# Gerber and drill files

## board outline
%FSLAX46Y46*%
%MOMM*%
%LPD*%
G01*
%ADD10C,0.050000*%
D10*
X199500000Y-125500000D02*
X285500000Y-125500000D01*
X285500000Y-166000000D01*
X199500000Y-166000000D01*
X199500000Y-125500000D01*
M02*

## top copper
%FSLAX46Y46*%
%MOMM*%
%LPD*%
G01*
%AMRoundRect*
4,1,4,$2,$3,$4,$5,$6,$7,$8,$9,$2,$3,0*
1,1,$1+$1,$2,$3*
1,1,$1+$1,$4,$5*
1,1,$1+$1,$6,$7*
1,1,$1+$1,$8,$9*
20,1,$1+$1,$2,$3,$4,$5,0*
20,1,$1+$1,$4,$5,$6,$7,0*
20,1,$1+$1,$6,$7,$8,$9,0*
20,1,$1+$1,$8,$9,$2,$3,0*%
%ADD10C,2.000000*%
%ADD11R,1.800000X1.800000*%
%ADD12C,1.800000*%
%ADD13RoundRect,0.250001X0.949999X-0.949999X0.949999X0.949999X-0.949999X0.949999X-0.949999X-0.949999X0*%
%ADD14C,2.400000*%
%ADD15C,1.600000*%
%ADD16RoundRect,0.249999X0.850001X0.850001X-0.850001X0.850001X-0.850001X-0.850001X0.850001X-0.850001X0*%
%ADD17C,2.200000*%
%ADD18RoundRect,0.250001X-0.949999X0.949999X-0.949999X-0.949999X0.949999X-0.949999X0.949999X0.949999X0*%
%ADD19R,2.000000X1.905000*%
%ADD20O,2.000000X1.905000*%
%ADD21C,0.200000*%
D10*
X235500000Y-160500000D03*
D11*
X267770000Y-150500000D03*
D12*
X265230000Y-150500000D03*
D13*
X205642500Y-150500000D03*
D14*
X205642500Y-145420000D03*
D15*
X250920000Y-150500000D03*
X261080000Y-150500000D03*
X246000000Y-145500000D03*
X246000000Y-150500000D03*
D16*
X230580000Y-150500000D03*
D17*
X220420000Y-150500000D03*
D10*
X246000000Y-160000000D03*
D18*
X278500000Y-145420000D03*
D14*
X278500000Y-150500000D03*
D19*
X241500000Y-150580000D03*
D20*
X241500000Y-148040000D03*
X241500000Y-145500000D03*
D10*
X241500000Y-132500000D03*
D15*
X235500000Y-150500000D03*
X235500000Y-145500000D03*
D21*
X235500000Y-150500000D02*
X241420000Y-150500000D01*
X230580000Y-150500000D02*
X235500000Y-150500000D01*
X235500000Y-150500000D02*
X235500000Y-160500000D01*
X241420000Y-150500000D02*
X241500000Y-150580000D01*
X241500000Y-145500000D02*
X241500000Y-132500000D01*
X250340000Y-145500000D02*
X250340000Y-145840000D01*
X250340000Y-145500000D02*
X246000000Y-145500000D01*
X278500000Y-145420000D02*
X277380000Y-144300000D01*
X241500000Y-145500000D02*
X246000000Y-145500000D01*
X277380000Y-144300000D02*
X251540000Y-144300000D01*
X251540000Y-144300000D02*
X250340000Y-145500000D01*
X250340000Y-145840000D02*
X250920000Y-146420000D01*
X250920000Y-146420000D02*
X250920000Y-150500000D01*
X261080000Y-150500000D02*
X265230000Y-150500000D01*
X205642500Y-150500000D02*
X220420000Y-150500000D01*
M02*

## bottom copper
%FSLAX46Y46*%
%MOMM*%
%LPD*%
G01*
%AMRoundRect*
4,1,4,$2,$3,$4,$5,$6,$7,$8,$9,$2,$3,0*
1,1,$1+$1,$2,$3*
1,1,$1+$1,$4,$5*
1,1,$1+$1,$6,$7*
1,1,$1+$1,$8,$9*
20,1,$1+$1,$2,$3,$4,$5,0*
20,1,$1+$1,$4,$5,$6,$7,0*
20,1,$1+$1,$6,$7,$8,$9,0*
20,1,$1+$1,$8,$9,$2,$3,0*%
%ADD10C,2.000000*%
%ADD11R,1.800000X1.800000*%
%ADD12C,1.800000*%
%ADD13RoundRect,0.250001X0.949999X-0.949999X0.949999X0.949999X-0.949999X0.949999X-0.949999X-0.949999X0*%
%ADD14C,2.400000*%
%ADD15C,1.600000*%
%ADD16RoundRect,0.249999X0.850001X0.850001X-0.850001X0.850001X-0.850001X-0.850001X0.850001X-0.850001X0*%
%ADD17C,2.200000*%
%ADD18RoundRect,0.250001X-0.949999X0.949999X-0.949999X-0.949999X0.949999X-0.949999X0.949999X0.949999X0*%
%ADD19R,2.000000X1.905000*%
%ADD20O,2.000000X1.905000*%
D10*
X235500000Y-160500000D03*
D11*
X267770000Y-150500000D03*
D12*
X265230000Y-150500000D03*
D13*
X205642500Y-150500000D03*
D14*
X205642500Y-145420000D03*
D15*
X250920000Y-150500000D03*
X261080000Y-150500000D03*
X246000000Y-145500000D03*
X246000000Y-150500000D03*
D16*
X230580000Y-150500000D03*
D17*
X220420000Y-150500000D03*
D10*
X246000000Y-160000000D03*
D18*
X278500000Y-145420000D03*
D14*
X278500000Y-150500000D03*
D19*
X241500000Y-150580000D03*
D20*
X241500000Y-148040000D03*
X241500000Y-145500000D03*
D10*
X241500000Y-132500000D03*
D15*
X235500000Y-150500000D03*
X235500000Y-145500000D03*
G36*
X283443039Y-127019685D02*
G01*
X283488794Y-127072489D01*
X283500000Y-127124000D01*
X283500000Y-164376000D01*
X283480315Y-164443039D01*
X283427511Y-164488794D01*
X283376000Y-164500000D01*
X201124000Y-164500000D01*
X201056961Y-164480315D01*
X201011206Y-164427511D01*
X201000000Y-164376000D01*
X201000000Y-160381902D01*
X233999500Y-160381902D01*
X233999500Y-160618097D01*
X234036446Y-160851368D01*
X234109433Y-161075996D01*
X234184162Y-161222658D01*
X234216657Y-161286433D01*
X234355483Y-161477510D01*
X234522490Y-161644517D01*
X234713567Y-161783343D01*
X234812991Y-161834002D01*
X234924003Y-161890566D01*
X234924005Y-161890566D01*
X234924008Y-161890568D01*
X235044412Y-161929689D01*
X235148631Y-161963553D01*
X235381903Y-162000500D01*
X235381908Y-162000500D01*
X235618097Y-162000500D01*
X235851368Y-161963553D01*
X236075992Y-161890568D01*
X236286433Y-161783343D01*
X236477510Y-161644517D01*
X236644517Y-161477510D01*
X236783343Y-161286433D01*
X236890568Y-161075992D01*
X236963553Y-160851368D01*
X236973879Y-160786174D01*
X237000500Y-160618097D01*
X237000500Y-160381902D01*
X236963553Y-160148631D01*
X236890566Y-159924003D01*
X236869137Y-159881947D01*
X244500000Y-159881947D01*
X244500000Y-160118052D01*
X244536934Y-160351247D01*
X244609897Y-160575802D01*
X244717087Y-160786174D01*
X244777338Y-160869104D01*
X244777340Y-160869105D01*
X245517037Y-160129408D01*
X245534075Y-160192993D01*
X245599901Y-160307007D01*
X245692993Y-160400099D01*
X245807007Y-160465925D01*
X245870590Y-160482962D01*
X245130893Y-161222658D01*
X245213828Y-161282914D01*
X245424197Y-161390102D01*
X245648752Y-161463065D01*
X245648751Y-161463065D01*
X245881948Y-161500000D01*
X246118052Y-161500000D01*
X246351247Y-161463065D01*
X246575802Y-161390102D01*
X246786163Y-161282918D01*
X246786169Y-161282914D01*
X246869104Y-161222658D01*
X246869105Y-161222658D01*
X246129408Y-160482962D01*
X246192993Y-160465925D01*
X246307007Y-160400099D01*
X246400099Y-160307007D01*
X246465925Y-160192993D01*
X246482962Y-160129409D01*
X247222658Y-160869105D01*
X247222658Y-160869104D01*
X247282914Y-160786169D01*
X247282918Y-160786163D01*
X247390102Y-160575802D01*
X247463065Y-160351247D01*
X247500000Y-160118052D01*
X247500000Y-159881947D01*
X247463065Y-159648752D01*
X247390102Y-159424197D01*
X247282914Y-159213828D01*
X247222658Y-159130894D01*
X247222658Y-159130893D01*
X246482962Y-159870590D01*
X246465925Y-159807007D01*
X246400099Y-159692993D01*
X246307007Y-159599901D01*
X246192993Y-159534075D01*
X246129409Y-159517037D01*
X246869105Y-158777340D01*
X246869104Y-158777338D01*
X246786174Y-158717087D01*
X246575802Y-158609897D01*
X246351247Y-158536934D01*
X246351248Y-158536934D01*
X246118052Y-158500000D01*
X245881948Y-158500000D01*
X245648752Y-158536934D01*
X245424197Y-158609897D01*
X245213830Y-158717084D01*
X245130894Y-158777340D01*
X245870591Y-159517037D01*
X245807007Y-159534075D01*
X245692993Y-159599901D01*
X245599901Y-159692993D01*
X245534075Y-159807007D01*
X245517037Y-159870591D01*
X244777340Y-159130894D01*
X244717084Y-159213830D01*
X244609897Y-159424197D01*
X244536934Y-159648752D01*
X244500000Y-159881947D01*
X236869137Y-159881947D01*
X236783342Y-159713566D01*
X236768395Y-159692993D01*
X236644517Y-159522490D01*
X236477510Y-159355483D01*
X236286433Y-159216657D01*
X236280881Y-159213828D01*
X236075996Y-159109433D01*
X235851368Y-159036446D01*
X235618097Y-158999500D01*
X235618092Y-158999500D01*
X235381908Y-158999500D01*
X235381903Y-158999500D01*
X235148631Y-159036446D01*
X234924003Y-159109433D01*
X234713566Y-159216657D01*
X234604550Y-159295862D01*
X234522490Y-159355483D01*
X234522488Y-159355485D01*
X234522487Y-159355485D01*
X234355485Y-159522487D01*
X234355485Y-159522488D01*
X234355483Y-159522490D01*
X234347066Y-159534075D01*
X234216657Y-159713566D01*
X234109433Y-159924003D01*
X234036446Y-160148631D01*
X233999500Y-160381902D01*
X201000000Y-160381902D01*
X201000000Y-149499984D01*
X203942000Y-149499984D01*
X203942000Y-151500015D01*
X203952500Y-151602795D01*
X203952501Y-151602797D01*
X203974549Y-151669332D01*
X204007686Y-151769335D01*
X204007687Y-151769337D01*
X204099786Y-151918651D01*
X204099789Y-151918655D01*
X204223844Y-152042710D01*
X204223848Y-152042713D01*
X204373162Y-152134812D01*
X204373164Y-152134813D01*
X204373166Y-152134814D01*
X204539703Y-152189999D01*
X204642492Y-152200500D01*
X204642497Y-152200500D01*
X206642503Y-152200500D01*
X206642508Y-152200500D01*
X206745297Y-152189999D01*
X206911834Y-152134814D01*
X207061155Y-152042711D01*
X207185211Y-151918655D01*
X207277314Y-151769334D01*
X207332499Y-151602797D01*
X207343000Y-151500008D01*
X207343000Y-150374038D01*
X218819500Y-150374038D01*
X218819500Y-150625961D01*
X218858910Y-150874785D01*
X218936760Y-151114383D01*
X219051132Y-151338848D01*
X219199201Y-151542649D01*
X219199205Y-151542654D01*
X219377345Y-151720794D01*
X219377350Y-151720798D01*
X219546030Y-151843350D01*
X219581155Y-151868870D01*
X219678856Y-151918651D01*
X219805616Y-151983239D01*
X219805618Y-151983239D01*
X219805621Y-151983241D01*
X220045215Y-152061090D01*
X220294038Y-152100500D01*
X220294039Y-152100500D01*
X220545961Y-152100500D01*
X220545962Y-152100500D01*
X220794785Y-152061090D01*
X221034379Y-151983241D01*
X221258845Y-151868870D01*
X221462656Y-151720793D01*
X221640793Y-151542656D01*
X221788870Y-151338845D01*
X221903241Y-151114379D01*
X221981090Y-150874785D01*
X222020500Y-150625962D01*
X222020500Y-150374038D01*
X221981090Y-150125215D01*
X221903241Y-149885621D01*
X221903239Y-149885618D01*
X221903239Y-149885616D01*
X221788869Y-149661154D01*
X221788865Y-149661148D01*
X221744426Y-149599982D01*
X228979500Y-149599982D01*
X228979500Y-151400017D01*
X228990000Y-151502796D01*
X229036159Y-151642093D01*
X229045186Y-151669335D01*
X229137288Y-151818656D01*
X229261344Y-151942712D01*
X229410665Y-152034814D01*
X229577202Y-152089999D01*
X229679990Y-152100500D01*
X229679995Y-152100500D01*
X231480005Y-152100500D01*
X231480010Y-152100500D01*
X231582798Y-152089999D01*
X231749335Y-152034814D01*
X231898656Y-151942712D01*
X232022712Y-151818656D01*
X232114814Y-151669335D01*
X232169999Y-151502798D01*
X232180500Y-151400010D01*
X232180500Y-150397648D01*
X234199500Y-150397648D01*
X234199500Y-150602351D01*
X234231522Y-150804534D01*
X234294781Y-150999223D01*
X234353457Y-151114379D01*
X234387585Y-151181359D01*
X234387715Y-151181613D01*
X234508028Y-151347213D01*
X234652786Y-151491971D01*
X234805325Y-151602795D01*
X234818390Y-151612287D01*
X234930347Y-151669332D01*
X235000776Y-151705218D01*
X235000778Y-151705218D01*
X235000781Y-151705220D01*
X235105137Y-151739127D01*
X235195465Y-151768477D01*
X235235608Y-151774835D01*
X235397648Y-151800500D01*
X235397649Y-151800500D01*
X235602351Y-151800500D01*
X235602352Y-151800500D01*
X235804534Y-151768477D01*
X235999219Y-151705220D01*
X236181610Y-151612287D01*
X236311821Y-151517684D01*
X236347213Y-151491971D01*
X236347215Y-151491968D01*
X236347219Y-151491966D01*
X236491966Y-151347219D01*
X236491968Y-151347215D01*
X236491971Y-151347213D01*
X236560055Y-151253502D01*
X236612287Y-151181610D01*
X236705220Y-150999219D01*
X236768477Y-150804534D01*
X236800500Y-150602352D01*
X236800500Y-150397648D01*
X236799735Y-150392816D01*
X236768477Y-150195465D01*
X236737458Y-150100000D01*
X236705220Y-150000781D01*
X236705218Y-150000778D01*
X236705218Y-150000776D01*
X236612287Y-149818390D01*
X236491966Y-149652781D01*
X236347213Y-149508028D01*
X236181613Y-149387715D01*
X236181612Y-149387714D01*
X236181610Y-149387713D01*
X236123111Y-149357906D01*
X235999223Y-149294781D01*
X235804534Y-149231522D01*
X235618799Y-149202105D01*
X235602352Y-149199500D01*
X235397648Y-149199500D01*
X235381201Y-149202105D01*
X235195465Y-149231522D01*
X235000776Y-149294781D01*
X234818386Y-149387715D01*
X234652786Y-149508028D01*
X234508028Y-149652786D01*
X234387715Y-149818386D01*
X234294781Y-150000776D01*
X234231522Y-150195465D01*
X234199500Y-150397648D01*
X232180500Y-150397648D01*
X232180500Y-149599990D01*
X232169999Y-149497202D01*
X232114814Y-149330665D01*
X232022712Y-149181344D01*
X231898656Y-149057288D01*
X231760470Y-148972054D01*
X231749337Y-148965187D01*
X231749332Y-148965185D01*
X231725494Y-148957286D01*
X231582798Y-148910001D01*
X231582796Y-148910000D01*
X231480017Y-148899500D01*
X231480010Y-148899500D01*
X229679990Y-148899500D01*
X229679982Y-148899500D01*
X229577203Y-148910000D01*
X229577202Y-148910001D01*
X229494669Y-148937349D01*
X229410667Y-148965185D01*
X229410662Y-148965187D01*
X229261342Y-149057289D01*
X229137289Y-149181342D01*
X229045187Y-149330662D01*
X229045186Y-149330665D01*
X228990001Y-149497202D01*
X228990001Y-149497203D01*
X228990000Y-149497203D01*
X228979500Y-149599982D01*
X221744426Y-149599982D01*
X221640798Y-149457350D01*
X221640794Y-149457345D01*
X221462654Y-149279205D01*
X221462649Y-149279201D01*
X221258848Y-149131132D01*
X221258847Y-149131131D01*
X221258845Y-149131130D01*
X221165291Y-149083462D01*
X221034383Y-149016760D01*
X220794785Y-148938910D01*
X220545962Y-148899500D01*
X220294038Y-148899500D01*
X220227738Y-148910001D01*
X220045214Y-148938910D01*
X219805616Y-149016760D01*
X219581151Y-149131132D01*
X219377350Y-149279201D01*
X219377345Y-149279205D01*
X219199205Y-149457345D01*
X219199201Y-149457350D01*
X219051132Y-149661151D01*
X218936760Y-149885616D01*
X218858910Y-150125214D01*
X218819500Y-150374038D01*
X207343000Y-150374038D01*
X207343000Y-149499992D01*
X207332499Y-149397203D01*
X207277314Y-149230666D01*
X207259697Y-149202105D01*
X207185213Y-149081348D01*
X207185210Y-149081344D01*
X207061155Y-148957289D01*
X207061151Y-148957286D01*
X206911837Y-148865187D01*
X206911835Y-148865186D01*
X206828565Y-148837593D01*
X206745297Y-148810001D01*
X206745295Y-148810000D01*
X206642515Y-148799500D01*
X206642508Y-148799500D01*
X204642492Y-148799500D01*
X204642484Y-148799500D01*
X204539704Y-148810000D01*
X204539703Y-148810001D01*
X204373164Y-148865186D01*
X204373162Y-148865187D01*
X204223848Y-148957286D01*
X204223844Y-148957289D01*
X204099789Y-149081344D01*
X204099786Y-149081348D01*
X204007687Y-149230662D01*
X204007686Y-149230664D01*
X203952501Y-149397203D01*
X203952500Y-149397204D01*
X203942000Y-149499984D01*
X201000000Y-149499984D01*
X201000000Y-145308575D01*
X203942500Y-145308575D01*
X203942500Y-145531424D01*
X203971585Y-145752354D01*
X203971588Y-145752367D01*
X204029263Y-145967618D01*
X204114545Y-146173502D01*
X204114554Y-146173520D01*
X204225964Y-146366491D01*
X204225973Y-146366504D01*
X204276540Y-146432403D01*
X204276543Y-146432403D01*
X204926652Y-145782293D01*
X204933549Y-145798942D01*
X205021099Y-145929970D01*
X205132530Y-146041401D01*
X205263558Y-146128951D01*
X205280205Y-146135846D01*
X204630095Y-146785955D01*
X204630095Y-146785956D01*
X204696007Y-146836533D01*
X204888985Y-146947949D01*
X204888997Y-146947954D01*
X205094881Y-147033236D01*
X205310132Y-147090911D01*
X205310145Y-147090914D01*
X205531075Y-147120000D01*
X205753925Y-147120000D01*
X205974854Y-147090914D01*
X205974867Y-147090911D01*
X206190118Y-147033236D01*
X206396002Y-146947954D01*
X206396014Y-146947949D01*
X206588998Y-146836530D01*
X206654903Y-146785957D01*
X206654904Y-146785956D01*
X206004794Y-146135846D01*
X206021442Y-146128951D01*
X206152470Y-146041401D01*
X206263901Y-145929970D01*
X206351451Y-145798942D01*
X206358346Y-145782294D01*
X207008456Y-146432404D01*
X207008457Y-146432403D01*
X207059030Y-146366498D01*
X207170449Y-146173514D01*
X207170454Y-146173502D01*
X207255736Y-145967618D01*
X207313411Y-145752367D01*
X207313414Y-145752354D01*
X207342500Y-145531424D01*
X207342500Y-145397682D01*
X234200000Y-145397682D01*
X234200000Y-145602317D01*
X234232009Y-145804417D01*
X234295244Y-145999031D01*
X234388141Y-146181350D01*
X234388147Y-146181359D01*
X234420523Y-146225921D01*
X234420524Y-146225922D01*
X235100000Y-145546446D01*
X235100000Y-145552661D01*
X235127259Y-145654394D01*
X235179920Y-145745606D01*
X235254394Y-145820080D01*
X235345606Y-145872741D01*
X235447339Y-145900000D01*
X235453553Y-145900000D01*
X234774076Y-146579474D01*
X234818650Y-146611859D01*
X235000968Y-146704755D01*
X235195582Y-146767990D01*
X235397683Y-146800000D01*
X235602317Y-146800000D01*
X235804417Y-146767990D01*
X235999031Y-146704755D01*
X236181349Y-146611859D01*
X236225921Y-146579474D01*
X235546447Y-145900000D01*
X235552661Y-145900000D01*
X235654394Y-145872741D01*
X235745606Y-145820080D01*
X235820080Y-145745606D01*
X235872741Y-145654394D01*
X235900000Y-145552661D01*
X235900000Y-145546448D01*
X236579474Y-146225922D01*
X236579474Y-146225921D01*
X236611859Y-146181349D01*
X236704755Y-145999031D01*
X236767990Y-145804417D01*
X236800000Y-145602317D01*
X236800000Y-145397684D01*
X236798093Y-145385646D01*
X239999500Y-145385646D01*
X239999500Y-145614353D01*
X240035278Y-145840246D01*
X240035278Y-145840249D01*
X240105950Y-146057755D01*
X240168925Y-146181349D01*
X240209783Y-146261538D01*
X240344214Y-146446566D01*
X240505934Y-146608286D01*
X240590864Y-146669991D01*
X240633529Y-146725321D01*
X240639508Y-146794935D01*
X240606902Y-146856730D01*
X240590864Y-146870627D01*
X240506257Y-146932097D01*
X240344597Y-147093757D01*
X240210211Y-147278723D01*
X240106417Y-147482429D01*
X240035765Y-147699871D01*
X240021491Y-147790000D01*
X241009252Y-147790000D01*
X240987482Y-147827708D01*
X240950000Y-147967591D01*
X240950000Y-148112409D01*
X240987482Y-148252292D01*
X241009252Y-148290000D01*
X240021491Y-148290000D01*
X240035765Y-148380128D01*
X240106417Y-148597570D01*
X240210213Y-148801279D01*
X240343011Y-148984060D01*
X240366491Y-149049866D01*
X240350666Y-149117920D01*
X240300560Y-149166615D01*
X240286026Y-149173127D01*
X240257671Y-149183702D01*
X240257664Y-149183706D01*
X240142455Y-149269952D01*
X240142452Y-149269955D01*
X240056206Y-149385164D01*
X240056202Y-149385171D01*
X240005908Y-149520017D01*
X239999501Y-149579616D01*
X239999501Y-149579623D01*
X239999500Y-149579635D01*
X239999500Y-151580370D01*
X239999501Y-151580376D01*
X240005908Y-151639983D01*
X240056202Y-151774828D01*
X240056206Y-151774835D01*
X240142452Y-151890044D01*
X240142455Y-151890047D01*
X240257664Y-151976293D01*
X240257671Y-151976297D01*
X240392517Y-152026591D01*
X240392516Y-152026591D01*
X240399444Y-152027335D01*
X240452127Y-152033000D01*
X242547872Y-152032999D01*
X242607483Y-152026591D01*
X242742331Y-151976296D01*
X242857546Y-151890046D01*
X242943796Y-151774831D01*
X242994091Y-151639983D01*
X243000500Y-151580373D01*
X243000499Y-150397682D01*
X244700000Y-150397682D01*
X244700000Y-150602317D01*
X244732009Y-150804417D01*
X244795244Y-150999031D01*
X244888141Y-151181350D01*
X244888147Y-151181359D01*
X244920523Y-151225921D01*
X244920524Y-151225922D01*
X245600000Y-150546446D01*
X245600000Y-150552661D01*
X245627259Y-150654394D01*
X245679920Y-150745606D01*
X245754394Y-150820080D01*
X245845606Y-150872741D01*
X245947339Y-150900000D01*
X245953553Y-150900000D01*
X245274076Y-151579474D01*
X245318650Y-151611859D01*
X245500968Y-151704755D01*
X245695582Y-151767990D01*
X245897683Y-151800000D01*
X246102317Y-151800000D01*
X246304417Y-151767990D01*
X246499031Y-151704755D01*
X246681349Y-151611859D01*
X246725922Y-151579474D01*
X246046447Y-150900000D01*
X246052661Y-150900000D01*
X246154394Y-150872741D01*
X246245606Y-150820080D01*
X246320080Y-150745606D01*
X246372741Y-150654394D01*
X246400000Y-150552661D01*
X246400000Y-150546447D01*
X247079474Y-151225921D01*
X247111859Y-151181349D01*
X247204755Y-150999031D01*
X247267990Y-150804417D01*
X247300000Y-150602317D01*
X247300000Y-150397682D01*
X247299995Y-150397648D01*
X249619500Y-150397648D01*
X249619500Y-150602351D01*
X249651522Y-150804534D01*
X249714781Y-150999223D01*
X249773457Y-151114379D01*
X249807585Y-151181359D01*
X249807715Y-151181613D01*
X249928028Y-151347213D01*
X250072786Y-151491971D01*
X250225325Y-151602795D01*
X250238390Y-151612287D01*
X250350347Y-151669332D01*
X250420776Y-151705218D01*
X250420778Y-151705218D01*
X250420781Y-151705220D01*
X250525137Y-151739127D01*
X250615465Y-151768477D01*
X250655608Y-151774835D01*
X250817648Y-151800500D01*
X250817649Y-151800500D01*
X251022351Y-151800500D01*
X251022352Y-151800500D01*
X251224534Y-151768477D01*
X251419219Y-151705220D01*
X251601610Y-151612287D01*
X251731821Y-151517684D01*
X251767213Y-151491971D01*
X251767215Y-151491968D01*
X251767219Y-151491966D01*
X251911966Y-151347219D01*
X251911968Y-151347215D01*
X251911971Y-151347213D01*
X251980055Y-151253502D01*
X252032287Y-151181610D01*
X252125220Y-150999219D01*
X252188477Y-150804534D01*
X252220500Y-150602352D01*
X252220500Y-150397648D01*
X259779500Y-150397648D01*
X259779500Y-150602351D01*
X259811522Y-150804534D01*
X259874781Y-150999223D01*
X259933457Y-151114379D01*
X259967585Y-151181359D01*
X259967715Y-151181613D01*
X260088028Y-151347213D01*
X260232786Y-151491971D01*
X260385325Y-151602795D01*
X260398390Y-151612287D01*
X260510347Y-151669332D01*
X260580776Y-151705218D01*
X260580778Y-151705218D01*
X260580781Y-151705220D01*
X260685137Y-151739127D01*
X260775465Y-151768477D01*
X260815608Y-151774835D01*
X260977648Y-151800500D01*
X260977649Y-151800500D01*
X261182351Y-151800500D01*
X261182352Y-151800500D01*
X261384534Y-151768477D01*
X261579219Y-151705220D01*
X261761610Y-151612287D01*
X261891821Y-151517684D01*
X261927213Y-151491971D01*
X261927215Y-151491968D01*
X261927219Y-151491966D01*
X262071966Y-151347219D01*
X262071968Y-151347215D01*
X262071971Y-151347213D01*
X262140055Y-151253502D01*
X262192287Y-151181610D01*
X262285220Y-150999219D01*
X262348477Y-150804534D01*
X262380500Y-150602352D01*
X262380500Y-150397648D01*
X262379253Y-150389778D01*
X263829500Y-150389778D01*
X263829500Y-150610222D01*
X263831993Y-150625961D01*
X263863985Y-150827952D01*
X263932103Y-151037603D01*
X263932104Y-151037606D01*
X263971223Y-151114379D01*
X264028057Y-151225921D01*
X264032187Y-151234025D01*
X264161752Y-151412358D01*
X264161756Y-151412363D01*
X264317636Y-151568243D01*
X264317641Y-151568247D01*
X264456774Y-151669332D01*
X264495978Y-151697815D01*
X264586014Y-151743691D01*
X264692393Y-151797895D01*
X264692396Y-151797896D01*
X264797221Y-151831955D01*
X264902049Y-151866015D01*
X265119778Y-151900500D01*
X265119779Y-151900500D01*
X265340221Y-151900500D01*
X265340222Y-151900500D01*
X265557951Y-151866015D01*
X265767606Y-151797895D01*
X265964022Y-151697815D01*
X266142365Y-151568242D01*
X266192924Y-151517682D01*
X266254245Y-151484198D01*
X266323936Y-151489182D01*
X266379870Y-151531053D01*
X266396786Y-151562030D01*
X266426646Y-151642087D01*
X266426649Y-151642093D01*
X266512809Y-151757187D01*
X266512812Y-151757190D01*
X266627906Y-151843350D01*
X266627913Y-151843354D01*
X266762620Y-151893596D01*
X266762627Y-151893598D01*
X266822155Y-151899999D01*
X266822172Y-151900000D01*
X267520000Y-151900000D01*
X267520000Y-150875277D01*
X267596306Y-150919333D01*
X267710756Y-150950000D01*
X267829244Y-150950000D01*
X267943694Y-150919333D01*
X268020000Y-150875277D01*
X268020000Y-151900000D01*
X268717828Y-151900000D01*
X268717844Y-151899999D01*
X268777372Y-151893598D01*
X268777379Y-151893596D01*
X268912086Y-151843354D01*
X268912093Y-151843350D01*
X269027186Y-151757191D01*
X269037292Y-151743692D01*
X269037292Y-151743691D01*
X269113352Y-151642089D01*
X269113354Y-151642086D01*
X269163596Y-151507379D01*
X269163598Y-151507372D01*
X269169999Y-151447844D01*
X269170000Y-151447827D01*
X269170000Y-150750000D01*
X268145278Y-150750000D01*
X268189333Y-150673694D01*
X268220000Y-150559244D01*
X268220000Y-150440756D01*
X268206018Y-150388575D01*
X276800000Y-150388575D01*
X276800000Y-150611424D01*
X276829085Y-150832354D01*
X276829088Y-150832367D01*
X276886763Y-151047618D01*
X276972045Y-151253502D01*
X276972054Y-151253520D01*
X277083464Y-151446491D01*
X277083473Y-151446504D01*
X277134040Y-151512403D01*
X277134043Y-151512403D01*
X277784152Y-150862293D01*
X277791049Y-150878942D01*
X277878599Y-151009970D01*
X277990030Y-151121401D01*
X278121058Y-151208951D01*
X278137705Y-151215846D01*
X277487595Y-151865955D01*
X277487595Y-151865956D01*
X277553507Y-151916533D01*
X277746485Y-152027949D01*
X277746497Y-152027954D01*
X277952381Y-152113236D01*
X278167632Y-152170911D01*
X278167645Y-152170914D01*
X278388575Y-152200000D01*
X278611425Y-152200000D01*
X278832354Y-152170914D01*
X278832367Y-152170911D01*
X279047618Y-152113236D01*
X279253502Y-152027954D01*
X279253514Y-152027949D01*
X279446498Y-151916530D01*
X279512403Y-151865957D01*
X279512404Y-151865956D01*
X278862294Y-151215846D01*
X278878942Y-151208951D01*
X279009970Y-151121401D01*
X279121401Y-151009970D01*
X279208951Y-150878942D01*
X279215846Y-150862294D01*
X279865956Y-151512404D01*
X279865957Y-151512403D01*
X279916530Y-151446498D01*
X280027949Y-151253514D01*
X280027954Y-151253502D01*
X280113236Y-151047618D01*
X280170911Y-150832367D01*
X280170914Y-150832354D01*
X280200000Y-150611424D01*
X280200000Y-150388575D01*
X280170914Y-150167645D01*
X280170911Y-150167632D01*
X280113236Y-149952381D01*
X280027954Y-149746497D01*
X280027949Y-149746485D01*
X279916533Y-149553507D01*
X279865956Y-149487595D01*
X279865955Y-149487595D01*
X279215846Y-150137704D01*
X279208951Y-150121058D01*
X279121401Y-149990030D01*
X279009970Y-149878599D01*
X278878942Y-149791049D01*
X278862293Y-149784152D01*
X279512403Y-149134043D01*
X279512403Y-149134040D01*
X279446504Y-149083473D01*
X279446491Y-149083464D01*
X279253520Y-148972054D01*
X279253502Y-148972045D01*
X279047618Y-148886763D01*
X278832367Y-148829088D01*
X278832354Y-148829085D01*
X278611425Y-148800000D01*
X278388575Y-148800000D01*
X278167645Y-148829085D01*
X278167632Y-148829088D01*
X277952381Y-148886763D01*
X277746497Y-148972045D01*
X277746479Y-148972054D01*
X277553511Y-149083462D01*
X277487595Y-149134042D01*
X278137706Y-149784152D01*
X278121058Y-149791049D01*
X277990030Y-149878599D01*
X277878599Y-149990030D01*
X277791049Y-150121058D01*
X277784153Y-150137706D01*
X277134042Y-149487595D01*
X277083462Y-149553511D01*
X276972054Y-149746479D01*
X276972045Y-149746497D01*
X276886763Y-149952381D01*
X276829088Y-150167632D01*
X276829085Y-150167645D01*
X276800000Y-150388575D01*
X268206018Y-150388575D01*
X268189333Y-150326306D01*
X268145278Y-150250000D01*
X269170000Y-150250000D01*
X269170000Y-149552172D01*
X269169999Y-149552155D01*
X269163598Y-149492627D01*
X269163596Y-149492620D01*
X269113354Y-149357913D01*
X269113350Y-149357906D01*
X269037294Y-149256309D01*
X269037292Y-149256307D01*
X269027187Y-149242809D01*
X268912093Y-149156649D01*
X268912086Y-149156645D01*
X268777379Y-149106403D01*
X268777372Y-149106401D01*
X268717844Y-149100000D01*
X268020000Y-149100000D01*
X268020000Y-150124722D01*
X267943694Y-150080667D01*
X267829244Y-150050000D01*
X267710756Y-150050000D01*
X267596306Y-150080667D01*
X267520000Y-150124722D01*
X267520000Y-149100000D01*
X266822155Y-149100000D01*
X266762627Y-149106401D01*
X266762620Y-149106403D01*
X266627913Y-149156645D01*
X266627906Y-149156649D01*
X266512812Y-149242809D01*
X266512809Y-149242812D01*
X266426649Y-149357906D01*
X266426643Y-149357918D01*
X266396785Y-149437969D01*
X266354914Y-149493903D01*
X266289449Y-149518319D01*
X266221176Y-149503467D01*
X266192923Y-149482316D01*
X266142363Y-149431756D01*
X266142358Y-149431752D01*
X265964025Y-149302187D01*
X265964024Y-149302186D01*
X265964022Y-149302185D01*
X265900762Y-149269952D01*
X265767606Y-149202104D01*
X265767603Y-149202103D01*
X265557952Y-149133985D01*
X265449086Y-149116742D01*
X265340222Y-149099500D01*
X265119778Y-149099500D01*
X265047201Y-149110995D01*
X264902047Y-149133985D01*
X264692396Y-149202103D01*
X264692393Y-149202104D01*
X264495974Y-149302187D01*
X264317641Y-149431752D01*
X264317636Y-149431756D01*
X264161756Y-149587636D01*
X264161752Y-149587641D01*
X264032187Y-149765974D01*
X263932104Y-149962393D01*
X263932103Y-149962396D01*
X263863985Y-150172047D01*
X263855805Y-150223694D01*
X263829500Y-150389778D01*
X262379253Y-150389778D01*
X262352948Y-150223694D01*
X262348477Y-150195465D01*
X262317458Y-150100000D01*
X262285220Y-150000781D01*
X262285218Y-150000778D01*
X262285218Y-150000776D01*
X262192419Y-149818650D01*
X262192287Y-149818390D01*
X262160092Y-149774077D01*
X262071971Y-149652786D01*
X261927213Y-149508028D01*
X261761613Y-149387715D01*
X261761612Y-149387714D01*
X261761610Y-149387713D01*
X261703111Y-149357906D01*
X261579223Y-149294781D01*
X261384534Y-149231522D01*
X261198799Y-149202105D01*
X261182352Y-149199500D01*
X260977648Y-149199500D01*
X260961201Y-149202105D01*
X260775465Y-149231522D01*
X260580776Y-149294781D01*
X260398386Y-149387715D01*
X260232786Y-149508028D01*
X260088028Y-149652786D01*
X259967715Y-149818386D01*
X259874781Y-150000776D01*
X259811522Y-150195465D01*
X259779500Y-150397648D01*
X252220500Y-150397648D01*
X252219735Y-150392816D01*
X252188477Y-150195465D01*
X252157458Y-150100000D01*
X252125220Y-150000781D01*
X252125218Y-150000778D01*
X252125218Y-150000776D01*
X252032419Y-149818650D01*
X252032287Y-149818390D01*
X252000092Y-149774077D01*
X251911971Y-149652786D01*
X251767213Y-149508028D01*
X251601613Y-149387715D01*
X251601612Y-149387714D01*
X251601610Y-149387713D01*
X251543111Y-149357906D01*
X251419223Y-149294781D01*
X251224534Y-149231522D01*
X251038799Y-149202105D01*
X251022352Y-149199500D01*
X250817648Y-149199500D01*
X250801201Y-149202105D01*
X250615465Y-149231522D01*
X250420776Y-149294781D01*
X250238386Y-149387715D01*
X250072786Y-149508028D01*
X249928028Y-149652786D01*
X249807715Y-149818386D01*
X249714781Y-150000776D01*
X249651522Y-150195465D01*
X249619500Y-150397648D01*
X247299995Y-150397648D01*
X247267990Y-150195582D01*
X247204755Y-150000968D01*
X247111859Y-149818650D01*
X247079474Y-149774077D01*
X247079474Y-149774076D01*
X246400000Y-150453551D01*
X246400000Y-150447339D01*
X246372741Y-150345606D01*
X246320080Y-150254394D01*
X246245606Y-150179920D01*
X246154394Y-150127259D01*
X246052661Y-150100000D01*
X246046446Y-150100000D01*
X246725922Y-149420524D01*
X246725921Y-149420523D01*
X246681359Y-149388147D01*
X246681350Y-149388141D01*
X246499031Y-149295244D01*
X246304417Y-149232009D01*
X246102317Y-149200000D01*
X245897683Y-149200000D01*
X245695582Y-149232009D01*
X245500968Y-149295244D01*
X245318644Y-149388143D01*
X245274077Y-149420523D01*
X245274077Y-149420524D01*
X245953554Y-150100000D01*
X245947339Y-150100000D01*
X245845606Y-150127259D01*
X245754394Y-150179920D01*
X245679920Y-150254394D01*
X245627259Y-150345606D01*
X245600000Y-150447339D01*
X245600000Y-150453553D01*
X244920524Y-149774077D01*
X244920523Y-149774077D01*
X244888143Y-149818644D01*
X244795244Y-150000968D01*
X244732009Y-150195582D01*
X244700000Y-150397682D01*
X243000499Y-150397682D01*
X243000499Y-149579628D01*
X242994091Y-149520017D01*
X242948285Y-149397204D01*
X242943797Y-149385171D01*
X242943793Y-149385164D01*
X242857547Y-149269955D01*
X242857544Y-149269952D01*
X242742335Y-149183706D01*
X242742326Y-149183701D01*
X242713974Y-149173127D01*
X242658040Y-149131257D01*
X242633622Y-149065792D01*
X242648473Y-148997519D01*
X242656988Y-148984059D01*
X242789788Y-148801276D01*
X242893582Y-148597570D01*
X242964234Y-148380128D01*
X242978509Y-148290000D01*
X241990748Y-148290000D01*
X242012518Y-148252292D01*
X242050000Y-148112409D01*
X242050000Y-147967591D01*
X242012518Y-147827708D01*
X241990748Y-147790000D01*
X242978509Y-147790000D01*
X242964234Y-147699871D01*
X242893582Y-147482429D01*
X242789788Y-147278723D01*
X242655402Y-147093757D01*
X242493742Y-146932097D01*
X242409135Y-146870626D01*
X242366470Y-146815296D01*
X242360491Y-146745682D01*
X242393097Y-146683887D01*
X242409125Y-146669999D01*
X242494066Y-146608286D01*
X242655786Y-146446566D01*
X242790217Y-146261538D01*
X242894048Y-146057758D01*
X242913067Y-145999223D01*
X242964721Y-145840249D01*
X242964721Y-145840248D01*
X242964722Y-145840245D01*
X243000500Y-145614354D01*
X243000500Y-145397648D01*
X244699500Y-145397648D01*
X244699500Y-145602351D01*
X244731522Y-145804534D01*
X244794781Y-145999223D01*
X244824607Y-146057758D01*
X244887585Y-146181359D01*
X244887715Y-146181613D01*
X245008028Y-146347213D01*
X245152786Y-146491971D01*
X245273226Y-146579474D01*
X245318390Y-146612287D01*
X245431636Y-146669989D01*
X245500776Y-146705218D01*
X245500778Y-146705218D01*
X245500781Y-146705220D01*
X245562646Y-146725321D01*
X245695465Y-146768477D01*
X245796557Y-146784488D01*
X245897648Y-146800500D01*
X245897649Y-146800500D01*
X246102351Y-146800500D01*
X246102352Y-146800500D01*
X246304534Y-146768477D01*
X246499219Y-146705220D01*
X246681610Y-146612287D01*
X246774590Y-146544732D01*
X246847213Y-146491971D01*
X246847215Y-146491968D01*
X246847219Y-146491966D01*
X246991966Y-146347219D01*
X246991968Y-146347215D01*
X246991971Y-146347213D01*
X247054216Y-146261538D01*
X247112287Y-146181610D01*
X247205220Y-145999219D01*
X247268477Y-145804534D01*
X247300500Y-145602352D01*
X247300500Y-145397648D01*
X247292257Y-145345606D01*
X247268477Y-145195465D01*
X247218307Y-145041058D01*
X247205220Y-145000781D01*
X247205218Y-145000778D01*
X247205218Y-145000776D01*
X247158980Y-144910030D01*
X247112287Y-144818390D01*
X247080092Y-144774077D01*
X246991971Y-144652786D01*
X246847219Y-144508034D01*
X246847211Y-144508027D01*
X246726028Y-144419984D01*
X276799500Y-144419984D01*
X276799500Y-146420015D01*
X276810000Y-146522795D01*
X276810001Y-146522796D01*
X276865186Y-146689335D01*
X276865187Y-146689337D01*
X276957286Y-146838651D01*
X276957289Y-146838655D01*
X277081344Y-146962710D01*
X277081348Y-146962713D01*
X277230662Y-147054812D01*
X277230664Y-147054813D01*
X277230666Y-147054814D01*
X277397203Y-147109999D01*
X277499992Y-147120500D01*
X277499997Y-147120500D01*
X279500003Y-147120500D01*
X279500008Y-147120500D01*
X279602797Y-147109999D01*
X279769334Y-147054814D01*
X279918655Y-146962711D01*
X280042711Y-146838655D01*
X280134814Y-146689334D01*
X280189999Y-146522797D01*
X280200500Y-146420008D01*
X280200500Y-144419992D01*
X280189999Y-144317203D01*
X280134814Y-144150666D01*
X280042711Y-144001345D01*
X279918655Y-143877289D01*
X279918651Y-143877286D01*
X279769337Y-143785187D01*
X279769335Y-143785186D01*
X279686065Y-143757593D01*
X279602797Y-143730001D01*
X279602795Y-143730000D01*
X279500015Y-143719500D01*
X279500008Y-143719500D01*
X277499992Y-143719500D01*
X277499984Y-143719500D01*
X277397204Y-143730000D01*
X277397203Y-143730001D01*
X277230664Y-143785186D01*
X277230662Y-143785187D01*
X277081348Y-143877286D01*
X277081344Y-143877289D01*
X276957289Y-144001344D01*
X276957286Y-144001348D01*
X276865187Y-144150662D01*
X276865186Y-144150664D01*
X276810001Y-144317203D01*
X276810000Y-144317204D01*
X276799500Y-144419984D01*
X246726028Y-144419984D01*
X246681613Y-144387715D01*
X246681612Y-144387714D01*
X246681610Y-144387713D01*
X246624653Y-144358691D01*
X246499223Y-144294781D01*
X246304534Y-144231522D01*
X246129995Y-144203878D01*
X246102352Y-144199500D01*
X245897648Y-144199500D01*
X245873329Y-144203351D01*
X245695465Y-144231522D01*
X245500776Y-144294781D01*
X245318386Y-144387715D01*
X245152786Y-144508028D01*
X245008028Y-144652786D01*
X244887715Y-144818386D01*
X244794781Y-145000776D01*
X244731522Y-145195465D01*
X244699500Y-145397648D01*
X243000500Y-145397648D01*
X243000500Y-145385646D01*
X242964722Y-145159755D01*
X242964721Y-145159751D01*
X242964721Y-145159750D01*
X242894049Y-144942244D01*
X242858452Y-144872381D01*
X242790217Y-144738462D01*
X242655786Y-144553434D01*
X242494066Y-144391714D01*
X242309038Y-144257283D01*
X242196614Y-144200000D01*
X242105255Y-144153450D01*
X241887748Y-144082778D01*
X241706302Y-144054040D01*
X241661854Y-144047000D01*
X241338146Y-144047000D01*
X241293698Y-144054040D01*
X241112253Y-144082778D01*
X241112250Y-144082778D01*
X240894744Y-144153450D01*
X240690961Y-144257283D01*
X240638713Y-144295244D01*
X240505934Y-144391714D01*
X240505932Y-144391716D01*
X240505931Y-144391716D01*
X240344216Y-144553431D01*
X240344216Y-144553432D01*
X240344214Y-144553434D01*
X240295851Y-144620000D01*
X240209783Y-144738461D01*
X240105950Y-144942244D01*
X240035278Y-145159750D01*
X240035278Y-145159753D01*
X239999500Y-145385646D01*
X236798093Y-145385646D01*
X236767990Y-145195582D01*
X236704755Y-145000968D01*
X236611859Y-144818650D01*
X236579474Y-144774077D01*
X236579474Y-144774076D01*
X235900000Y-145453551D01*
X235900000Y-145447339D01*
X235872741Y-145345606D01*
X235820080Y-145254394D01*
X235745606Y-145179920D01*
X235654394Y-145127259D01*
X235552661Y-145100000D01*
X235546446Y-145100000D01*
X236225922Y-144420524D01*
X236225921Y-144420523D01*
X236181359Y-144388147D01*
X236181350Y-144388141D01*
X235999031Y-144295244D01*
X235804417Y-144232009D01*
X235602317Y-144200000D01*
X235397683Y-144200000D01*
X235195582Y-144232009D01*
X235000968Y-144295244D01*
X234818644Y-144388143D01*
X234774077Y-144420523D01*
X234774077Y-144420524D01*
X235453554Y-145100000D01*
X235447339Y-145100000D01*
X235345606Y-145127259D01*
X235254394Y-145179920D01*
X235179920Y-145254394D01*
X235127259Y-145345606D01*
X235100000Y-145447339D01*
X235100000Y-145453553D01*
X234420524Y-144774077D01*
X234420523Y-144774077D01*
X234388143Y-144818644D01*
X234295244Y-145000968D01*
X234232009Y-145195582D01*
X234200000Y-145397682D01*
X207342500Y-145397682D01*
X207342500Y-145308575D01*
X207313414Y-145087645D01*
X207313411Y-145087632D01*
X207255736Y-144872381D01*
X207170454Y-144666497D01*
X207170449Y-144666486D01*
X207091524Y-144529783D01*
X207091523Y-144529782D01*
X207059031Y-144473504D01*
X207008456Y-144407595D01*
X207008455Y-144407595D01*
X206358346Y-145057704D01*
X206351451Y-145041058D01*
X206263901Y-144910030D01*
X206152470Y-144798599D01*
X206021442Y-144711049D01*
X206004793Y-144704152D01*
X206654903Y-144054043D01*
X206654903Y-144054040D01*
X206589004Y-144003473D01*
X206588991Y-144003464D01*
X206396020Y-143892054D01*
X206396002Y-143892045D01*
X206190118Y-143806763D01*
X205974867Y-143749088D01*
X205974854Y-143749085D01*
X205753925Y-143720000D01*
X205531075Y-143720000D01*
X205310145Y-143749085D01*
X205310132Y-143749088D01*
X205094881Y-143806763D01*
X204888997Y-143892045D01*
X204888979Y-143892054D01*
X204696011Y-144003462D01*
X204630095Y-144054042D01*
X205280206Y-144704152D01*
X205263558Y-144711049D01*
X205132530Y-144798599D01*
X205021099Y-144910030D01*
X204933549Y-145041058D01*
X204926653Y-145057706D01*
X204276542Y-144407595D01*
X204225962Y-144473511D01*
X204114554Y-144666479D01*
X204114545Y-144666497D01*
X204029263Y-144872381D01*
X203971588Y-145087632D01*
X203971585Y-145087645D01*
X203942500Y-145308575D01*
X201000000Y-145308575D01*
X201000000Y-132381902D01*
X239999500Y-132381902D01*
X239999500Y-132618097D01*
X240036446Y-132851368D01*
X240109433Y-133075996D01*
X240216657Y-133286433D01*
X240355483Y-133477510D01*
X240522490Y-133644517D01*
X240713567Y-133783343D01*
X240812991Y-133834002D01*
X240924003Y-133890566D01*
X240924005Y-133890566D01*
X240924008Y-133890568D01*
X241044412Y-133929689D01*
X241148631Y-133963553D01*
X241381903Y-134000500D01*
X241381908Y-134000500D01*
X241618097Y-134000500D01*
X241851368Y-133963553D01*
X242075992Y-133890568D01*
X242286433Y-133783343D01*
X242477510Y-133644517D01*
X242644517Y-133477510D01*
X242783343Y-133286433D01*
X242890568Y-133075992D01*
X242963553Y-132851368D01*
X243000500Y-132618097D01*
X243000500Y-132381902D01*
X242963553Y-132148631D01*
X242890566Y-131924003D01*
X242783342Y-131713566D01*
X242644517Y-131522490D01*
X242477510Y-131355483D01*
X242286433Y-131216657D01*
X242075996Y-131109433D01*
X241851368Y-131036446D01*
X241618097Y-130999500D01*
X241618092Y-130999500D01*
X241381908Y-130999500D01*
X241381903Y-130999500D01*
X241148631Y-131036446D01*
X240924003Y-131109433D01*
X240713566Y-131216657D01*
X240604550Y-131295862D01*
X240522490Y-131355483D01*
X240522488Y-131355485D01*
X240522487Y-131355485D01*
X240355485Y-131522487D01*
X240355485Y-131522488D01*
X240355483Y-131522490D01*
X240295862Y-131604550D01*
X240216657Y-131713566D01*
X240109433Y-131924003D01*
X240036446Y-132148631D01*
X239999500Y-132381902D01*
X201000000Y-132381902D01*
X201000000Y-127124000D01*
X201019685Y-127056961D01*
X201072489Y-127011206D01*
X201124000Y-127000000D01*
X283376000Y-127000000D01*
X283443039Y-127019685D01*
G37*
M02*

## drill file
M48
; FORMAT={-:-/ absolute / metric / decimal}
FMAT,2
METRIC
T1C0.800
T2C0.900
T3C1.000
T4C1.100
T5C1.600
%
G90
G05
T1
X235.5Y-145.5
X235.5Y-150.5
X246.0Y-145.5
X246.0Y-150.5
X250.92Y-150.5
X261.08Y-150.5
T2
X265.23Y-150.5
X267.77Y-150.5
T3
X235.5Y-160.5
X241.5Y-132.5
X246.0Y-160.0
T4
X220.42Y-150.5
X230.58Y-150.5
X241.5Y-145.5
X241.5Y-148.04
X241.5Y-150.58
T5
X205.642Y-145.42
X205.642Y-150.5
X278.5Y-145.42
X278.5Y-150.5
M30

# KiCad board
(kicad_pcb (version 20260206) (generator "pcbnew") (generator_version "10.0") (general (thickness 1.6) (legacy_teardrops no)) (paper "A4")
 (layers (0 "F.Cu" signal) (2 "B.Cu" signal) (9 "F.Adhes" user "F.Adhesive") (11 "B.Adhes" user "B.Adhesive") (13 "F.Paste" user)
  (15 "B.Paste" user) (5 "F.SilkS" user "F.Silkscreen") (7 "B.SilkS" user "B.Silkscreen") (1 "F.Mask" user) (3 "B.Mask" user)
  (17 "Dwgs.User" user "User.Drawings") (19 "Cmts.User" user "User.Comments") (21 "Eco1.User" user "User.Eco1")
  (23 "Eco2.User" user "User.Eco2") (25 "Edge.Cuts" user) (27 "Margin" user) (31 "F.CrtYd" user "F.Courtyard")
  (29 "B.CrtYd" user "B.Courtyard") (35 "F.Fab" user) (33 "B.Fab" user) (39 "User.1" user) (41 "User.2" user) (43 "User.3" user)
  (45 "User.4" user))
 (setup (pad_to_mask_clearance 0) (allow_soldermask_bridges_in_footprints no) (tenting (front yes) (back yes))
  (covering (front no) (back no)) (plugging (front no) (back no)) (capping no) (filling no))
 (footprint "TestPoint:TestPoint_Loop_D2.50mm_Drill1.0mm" (layer "F.Cu") (at 235.5 160.5)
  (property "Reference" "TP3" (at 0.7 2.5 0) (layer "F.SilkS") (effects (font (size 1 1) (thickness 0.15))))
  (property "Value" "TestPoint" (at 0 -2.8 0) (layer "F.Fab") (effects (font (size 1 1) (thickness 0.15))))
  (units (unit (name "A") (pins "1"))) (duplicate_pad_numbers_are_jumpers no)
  (pad "1" thru_hole circle (at 0 0) (size 2 2) (drill 1) (layers "*.Cu" "*.Mask") (remove_unused_layers no) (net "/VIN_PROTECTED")))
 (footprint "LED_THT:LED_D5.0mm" (layer "F.Cu") (at 267.77 150.5 180)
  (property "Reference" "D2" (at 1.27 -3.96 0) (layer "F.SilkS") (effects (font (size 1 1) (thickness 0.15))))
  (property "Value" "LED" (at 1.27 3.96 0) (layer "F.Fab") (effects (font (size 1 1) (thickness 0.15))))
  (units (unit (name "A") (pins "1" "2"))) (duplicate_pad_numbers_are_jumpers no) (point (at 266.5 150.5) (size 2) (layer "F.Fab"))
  (pad "1" thru_hole rect (at 0 0 180) (size 1.8 1.8) (drill 0.9) (layers "*.Cu" "*.Mask") (remove_unused_layers no) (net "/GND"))
  (pad "2" thru_hole circle (at 2.54 0 180) (size 1.8 1.8) (drill 0.9) (layers "*.Cu" "*.Mask") (remove_unused_layers no) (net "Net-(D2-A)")))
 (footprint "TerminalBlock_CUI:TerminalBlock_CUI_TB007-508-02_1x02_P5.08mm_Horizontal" (layer "F.Cu") (at 205.6425 150.5 90)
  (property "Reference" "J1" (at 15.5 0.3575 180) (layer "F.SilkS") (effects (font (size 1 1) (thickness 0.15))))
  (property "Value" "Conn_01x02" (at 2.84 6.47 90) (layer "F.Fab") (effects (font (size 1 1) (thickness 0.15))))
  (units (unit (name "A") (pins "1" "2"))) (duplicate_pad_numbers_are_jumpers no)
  (pad "1" thru_hole roundrect (at 0 0 90) (size 2.4 2.4) (drill 1.6) (layers "*.Cu" "*.Mask") (remove_unused_layers no)
   (roundrect_rratio 0.104167) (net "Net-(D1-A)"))
  (pad "2" thru_hole circle (at 5.08 0 90) (size 2.4 2.4) (drill 1.6) (layers "*.Cu" "*.Mask") (remove_unused_layers no) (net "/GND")))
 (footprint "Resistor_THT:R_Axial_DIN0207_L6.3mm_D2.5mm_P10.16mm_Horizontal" (layer "F.Cu") (at 250.92 150.5)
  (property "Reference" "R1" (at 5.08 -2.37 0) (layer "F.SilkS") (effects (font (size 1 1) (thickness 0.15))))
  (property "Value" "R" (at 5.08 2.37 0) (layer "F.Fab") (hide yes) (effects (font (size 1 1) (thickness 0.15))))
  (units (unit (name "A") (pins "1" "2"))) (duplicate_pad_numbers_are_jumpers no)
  (pad "1" thru_hole circle (at 0 0) (size 1.6 1.6) (drill 0.8) (layers "*.Cu" "*.Mask") (remove_unused_layers no) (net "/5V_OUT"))
  (pad "2" thru_hole circle (at 10.16 0) (size 1.6 1.6) (drill 0.8) (layers "*.Cu" "*.Mask") (remove_unused_layers no) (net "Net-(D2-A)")))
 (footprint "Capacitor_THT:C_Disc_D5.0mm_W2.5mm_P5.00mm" (layer "F.Cu") (at 246 145.5 -90)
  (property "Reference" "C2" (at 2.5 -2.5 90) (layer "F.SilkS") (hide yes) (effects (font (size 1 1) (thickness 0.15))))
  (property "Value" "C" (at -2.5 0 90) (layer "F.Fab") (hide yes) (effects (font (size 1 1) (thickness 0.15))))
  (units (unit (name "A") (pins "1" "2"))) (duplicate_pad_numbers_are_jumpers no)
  (pad "1" thru_hole circle (at 0 0 270) (size 1.6 1.6) (drill 0.8) (layers "*.Cu" "*.Mask") (remove_unused_layers no) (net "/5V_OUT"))
  (pad "2" thru_hole circle (at 5 0 270) (size 1.6 1.6) (drill 0.8) (layers "*.Cu" "*.Mask") (remove_unused_layers no) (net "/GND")))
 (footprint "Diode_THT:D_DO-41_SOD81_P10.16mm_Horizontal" (layer "F.Cu") (at 230.58 150.5 180)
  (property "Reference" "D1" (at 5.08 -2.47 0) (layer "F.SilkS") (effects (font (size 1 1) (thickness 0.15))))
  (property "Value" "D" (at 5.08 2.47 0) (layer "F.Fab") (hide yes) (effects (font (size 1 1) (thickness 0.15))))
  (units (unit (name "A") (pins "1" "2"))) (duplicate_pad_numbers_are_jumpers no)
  (pad "1" thru_hole roundrect (at 0 0 180) (size 2.2 2.2) (drill 1.1) (layers "*.Cu" "*.Mask") (remove_unused_layers no)
   (roundrect_rratio 0.113636) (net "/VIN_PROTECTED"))
  (pad "2" thru_hole circle (at 10.16 0 180) (size 2.2 2.2) (drill 1.1) (layers "*.Cu" "*.Mask") (remove_unused_layers no)
   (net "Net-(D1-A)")))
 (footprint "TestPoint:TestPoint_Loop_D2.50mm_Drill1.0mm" (layer "F.Cu") (at 246 160)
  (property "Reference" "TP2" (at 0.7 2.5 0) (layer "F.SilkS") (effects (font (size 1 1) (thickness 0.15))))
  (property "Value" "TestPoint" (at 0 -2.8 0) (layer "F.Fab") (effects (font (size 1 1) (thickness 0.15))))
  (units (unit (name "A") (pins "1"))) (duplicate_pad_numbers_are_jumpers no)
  (pad "1" thru_hole circle (at 0 0) (size 2 2) (drill 1) (layers "*.Cu" "*.Mask") (remove_unused_layers no) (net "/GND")))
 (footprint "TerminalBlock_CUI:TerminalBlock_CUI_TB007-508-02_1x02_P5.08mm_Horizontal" (layer "F.Cu") (at 278.5 145.42 -90)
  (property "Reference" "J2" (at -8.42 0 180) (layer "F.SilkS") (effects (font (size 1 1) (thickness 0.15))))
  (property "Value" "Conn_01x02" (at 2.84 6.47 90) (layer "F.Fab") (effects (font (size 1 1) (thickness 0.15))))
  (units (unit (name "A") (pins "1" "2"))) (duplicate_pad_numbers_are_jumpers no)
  (pad "1" thru_hole roundrect (at 0 0 270) (size 2.4 2.4) (drill 1.6) (layers "*.Cu" "*.Mask") (remove_unused_layers no)
   (roundrect_rratio 0.104167) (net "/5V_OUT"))
  (pad "2" thru_hole circle (at 5.08 0 270) (size 2.4 2.4) (drill 1.6) (layers "*.Cu" "*.Mask") (remove_unused_layers no) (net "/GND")))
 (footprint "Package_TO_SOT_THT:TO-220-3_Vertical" (layer "F.Cu") (at 241.5 150.58 90)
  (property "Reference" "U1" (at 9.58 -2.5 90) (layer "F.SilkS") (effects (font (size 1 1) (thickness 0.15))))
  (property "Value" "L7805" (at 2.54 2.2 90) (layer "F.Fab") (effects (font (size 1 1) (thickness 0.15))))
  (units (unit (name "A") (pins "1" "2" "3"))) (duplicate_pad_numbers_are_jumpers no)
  (pad "1" thru_hole rect (at 0 0 90) (size 1.905 2) (drill 1.1) (layers "*.Cu" "*.Mask") (remove_unused_layers no) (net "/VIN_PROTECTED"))
  (pad "2" thru_hole oval (at 2.54 0 90) (size 1.905 2) (drill 1.1) (layers "*.Cu" "*.Mask") (remove_unused_layers no) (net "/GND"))
  (pad "3" thru_hole oval (at 5.08 0 90) (size 1.905 2) (drill 1.1) (layers "*.Cu" "*.Mask") (remove_unused_layers no) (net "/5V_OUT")))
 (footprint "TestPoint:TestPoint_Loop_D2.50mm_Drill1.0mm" (layer "F.Cu") (at 241.5 132.5)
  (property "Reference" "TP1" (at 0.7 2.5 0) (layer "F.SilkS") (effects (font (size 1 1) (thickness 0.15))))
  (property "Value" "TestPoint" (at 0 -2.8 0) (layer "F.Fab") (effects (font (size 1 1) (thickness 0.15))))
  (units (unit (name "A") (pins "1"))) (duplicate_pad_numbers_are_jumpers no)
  (pad "1" thru_hole circle (at 0 0) (size 2 2) (drill 1) (layers "*.Cu" "*.Mask") (remove_unused_layers no) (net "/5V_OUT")))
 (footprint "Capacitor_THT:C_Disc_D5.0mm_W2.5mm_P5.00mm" (layer "F.Cu") (at 235.5 150.5 90)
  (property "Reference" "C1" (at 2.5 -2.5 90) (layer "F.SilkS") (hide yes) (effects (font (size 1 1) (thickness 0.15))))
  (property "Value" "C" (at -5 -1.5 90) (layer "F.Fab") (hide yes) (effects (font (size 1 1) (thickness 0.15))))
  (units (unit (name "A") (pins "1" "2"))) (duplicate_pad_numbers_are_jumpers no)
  (pad "1" thru_hole circle (at 0 0 90) (size 1.6 1.6) (drill 0.8) (layers "*.Cu" "*.Mask") (remove_unused_layers no) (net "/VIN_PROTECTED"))
  (pad "2" thru_hole circle (at 5 0 90) (size 1.6 1.6) (drill 0.8) (layers "*.Cu" "*.Mask") (remove_unused_layers no) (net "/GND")))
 (gr_rect (start 199.5 125.5) (end 285.5 166) (stroke (width 0.05) (type default)) (fill no) (layer "Edge.Cuts"))
 (segment (start 235.5 150.5) (end 241.42 150.5) (width 0.2) (layer "F.Cu") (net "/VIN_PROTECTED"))
 (segment (start 230.58 150.5) (end 235.5 150.5) (width 0.2) (layer "F.Cu") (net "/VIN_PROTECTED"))
 (segment (start 235.5 150.5) (end 235.5 160.5) (width 0.2) (layer "F.Cu") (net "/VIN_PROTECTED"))
 (segment (start 241.42 150.5) (end 241.5 150.58) (width 0.2) (layer "F.Cu") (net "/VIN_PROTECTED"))
 (segment (start 241.5 145.5) (end 241.5 132.5) (width 0.2) (layer "F.Cu") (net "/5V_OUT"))
 (segment (start 250.34 145.5) (end 250.34 145.84) (width 0.2) (layer "F.Cu") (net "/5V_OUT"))
 (segment (start 250.34 145.5) (end 246 145.5) (width 0.2) (layer "F.Cu") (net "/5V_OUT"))
 (segment (start 278.5 145.42) (end 277.38 144.3) (width 0.2) (layer "F.Cu") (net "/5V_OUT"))
 (segment (start 241.5 145.5) (end 246 145.5) (width 0.2) (layer "F.Cu") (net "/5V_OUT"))
 (segment (start 277.38 144.3) (end 251.54 144.3) (width 0.2) (layer "F.Cu") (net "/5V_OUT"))
 (segment (start 251.54 144.3) (end 250.34 145.5) (width 0.2) (layer "F.Cu") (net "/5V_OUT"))
 (segment (start 250.34 145.84) (end 250.92 146.42) (width 0.2) (layer "F.Cu") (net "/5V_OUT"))
 (segment (start 250.92 146.42) (end 250.92 150.5) (width 0.2) (layer "F.Cu") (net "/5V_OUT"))
 (segment (start 261.08 150.5) (end 265.23 150.5) (width 0.2) (layer "F.Cu") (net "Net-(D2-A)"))
 (segment (start 205.6425 150.5) (end 220.42 150.5) (width 0.2) (layer "F.Cu") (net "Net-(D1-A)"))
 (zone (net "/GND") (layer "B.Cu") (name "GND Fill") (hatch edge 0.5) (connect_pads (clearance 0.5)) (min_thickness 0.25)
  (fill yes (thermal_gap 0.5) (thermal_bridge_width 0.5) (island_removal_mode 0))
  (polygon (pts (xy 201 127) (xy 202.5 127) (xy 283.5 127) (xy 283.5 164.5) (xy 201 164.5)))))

